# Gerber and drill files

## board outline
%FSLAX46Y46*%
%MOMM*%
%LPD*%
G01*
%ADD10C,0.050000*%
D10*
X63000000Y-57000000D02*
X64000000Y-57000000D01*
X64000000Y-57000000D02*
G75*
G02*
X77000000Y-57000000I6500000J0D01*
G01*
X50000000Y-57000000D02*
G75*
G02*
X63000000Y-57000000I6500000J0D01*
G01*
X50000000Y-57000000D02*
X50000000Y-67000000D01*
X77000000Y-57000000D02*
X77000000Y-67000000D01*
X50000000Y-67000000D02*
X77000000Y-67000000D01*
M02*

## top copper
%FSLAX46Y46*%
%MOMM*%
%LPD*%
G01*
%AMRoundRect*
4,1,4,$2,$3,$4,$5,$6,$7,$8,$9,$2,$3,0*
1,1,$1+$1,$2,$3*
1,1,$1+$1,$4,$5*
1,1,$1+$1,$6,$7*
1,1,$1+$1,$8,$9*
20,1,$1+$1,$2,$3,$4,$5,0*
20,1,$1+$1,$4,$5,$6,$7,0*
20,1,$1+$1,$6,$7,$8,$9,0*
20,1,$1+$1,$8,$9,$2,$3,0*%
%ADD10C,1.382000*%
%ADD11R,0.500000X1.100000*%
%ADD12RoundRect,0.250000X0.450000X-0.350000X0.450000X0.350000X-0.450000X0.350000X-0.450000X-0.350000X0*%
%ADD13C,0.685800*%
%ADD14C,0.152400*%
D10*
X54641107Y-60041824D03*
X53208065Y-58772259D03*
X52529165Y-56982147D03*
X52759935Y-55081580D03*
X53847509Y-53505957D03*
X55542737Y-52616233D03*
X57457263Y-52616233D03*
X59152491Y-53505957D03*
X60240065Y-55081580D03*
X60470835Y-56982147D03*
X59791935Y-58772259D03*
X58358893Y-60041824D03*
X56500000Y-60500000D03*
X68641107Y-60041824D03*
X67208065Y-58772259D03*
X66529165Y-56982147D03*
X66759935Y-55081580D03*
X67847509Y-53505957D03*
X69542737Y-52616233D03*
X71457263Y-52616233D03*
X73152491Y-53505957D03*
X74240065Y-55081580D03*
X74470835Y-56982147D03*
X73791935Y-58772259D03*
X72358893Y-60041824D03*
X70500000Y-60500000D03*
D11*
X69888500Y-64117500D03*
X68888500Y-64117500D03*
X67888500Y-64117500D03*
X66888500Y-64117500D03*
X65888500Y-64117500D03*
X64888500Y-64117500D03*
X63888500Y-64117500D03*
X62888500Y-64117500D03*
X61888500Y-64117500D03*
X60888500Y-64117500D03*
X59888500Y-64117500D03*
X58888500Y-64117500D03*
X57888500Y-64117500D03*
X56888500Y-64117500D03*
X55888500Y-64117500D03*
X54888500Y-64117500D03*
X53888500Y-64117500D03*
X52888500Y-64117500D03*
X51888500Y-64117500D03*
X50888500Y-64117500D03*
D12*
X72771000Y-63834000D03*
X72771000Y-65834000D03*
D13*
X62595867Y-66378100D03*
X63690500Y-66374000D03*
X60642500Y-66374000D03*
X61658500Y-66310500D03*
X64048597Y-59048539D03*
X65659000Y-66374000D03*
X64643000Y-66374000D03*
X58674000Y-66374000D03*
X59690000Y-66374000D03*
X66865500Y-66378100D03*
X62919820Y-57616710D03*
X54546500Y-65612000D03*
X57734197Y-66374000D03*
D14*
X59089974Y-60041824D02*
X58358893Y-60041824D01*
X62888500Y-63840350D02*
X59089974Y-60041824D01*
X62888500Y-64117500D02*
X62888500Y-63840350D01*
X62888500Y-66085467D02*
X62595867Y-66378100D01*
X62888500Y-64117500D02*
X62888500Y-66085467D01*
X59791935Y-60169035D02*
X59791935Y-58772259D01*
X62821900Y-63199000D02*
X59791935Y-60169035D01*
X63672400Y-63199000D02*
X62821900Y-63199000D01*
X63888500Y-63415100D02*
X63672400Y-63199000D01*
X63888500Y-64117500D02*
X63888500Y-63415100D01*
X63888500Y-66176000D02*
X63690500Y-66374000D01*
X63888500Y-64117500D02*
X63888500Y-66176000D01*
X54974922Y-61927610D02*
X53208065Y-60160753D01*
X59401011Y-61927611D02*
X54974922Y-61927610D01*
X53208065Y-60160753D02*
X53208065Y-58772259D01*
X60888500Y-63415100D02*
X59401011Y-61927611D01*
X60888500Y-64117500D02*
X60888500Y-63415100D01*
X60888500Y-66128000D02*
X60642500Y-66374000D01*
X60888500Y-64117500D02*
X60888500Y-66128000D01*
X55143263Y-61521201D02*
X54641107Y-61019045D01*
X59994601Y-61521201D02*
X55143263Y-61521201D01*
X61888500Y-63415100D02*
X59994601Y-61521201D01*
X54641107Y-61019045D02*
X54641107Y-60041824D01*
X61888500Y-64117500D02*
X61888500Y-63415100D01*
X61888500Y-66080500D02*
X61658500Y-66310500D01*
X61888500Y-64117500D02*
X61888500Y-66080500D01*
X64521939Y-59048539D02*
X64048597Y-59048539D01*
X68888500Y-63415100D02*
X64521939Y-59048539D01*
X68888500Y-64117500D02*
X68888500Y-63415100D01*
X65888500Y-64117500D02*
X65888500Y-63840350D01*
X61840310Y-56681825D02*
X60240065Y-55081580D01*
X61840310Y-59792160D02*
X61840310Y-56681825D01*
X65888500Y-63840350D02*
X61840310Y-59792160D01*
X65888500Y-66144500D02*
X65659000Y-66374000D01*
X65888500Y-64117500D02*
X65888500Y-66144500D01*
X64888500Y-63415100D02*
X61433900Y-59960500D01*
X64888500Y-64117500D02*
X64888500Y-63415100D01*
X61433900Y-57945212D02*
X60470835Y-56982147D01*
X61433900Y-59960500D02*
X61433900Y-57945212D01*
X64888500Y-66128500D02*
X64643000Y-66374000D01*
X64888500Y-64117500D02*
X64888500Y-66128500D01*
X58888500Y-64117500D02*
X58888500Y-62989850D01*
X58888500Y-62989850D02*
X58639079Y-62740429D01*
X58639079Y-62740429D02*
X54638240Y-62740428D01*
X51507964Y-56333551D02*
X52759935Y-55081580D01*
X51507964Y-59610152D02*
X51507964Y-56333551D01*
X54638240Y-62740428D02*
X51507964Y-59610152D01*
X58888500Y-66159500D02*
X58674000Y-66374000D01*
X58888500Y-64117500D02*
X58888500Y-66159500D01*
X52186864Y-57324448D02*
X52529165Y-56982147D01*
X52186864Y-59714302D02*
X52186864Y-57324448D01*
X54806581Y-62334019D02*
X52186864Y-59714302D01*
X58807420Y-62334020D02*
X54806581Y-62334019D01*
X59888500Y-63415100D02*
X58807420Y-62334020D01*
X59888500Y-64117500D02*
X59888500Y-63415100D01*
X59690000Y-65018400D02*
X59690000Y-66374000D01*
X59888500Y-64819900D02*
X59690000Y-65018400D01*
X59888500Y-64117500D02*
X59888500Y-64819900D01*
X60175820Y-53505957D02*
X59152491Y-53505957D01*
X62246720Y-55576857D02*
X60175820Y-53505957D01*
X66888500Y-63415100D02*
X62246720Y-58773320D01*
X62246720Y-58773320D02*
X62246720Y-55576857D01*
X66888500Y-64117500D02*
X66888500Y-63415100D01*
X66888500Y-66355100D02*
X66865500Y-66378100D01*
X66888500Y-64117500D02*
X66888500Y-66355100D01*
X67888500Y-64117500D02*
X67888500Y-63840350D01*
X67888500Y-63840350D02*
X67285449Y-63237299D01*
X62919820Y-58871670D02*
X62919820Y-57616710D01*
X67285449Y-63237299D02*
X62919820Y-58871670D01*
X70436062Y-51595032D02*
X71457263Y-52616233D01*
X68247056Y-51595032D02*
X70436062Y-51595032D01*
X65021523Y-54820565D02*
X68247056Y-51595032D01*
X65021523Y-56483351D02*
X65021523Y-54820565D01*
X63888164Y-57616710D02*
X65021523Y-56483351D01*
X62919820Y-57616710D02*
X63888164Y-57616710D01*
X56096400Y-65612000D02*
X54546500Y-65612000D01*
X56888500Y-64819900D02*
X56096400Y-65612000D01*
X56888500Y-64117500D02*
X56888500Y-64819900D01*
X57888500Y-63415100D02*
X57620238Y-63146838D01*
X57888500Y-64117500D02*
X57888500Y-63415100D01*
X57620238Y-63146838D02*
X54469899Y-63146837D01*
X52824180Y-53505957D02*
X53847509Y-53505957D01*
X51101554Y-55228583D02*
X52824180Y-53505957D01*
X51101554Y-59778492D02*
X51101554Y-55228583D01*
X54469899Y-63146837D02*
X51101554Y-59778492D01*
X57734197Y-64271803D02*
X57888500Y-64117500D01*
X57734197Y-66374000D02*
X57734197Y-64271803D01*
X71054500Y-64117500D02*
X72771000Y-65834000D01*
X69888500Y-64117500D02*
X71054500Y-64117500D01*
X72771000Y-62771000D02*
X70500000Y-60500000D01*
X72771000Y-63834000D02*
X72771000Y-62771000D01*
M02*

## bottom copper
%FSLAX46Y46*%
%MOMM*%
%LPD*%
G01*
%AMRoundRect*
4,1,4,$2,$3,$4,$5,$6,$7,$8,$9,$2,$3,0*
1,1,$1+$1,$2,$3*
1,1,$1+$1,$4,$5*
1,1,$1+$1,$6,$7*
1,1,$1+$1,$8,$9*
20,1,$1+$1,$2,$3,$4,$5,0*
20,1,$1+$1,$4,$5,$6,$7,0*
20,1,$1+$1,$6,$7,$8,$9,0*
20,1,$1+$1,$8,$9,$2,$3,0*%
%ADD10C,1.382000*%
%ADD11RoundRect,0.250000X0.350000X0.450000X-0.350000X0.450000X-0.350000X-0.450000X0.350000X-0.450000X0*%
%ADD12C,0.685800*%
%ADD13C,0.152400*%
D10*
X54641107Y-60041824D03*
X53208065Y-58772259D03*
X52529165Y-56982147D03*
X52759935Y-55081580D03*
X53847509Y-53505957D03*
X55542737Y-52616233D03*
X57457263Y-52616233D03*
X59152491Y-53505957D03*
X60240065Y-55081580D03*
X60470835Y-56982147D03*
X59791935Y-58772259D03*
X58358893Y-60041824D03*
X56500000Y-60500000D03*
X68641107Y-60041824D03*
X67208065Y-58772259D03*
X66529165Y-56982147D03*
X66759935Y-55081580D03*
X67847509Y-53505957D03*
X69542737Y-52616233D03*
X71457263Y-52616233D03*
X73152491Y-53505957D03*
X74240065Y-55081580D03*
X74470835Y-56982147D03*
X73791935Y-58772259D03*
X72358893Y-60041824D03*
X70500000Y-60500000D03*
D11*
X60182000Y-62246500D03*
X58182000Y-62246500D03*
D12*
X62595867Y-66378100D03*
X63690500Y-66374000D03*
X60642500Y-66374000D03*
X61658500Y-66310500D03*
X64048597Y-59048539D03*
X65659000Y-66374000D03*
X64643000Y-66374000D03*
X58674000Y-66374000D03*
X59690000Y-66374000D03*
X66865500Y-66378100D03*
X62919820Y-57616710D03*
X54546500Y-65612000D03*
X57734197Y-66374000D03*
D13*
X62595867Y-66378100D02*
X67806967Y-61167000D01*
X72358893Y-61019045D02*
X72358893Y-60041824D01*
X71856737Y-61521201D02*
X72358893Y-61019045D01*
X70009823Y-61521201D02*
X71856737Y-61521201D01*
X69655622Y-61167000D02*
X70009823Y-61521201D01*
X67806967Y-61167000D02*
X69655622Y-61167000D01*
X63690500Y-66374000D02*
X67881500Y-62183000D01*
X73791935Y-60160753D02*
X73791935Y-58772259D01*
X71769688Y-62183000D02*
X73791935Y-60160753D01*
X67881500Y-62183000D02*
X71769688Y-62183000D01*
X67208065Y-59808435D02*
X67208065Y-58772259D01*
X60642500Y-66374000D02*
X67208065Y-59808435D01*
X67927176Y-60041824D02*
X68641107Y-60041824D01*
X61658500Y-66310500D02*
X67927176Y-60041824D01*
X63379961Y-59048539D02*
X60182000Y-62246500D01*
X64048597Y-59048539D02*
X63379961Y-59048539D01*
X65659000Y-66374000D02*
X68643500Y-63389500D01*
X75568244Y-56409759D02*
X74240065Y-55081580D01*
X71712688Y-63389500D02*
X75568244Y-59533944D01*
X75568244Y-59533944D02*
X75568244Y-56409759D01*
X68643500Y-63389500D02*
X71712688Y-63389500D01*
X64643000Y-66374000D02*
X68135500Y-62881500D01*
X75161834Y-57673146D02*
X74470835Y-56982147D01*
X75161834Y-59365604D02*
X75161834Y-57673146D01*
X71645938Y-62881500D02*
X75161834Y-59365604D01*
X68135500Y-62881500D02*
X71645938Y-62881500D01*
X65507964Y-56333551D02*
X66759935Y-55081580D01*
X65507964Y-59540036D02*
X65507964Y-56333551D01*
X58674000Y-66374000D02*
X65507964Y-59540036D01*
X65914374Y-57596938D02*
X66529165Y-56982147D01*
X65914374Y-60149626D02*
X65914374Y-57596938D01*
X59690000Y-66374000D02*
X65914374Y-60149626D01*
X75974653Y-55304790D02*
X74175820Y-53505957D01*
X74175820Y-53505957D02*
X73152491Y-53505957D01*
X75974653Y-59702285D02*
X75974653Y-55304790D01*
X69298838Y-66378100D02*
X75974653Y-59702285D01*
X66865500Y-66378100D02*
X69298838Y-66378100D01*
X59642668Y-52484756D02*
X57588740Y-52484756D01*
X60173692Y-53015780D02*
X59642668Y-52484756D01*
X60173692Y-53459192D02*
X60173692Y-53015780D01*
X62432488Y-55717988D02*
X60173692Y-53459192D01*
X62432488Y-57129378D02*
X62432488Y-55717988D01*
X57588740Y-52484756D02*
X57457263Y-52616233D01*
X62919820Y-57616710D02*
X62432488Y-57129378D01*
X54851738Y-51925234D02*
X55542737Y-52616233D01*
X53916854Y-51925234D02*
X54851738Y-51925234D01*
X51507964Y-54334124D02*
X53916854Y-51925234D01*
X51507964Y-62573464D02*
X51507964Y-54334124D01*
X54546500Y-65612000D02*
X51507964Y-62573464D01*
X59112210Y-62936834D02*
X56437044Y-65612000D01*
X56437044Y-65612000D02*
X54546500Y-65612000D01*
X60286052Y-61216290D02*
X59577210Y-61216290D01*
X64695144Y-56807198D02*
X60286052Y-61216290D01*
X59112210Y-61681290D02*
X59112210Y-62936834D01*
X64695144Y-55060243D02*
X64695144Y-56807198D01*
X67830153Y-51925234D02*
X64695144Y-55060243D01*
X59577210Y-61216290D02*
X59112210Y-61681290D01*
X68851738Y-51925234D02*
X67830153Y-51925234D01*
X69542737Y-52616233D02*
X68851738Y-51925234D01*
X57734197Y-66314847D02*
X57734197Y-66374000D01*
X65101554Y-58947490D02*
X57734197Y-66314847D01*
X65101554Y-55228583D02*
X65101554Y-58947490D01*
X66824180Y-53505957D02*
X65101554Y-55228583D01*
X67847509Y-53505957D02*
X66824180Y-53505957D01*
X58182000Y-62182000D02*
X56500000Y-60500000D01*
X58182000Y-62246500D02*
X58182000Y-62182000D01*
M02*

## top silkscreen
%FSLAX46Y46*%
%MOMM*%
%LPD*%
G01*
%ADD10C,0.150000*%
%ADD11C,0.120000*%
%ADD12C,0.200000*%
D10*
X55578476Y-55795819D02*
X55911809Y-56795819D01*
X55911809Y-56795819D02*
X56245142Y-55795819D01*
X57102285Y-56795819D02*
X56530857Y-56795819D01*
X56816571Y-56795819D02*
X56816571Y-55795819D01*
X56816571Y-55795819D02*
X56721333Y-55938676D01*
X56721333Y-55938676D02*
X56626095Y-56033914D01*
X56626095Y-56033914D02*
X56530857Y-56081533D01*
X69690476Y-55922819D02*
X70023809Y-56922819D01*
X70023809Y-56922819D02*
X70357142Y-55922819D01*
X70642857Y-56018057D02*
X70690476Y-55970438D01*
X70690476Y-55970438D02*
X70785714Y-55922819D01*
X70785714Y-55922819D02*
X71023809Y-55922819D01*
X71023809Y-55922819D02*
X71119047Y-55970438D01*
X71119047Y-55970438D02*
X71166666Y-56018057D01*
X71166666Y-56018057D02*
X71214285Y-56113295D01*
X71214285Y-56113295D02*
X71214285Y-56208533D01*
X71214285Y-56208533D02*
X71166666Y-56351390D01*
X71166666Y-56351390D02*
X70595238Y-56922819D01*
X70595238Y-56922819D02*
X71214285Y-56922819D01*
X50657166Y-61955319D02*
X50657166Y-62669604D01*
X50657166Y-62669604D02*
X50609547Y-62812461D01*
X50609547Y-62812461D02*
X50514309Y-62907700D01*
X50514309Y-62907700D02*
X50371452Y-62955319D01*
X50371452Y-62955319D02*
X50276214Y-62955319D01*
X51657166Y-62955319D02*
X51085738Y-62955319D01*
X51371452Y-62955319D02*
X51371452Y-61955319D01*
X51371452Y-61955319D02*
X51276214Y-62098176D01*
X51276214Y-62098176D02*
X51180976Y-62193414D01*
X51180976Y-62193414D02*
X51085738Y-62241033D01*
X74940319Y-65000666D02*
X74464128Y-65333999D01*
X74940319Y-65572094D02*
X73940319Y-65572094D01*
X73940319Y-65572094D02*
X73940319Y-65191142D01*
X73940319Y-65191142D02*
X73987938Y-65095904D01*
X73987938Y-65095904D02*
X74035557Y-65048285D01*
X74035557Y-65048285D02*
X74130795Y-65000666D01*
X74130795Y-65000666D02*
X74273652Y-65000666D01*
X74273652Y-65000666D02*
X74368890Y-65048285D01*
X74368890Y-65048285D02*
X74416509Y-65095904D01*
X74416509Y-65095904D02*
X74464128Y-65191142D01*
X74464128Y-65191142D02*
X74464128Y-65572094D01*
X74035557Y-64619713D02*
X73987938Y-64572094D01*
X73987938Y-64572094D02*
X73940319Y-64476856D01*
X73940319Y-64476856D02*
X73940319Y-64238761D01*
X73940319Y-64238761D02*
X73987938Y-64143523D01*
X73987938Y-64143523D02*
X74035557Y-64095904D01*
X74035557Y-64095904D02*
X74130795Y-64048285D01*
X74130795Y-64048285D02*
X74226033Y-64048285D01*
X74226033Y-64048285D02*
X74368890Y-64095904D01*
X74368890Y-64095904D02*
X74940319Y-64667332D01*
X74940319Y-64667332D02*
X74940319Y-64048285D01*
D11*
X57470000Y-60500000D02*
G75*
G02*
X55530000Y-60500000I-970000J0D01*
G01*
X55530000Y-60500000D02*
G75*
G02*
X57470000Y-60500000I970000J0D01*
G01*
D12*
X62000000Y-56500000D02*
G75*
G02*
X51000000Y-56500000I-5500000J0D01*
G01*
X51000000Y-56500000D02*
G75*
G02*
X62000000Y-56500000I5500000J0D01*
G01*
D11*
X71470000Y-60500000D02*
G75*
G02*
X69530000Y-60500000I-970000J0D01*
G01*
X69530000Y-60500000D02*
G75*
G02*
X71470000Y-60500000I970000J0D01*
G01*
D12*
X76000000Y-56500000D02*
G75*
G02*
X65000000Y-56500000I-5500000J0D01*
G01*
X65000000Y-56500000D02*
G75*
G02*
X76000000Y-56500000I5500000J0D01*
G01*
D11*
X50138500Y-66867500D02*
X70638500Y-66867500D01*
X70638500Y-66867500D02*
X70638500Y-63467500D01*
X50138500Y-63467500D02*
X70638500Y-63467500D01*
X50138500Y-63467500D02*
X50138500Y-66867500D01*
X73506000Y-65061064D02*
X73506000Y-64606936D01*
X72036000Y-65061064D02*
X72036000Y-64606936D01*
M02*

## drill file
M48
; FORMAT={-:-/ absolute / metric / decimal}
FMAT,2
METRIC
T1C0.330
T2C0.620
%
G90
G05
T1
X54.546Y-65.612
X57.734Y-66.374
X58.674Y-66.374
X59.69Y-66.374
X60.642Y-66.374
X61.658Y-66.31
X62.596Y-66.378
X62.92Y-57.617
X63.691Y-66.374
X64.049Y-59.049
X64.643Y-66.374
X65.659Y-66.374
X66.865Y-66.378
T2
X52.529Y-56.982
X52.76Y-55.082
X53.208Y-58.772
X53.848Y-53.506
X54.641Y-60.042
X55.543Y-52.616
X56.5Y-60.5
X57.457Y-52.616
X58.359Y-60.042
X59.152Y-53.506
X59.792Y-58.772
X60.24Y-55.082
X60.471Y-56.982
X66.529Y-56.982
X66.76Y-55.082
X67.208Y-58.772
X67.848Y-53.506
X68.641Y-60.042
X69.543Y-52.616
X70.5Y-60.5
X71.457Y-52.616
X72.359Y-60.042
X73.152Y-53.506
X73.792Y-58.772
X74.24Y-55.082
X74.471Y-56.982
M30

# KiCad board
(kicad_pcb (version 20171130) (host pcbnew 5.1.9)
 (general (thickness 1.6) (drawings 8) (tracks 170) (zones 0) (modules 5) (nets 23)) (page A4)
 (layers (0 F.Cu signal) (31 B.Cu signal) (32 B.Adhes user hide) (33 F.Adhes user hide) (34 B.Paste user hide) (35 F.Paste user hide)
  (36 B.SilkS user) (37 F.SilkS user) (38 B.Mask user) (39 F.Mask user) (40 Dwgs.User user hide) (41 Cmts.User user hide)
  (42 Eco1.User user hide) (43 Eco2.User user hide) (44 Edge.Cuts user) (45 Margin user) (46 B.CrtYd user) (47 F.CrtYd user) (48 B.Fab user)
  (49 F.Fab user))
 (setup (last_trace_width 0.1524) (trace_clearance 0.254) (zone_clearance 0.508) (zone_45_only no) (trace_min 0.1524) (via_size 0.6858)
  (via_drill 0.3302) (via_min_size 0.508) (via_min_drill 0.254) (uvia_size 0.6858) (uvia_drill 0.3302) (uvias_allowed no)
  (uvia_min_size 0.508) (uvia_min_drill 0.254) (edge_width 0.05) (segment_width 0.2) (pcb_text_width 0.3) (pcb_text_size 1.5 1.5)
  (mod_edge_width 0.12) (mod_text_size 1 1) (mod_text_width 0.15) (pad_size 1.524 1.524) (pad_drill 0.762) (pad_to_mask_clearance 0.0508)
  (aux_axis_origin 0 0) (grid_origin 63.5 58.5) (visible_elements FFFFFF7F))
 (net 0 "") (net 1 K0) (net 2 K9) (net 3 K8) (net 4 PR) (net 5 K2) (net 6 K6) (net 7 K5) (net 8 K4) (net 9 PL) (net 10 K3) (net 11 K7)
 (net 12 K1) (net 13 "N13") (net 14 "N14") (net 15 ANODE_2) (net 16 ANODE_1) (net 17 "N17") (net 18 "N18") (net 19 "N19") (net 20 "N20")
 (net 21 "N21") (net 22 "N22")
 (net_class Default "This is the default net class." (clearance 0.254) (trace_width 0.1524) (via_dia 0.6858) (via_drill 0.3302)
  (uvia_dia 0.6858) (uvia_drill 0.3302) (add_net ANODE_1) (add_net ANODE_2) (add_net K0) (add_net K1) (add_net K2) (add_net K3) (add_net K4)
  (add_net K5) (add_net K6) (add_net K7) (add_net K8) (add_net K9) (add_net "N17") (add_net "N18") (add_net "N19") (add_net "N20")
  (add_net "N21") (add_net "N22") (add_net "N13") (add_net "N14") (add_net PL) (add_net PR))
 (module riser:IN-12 (layer F.Cu) (at 56.5 56.5)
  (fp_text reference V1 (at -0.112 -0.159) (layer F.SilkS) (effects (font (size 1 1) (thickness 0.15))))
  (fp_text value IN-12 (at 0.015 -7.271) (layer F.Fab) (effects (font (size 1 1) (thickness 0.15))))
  (fp_circle (center 0 4) (end 0.97 4) (layer F.SilkS) (width 0.12))
  (fp_circle (center 0 0) (end 5.5 0) (layer F.SilkS) (width 0.2))
  (pad 13 thru_hole circle (at -1.858893 3.541824) (size 1.382 1.382) (drill 0.62) (layers *.Cu *.Mask) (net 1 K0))
  (pad 12 thru_hole circle (at -3.291935 2.272259) (size 1.382 1.382) (drill 0.62) (layers *.Cu *.Mask) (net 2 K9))
  (pad 11 thru_hole circle (at -3.970835 0.482147) (size 1.382 1.382) (drill 0.62) (layers *.Cu *.Mask) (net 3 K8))
  (pad 10 thru_hole circle (at -3.740065 -1.41842) (size 1.382 1.382) (drill 0.62) (layers *.Cu *.Mask) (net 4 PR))
  (pad 9 thru_hole circle (at -2.652491 -2.994043) (size 1.382 1.382) (drill 0.62) (layers *.Cu *.Mask) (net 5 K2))
  (pad 8 thru_hole circle (at -0.957263 -3.883767) (size 1.382 1.382) (drill 0.62) (layers *.Cu *.Mask) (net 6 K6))
  (pad 7 thru_hole circle (at 0.957263 -3.883767) (size 1.382 1.382) (drill 0.62) (layers *.Cu *.Mask) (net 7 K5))
  (pad 6 thru_hole circle (at 2.652491 -2.994043) (size 1.382 1.382) (drill 0.62) (layers *.Cu *.Mask) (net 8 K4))
  (pad 5 thru_hole circle (at 3.740065 -1.41842) (size 1.382 1.382) (drill 0.62) (layers *.Cu *.Mask) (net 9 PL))
  (pad 4 thru_hole circle (at 3.970835 0.482147) (size 1.382 1.382) (drill 0.62) (layers *.Cu *.Mask) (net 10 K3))
  (pad 3 thru_hole circle (at 3.291935 2.272259) (size 1.382 1.382) (drill 0.62) (layers *.Cu *.Mask) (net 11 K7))
  (pad 2 thru_hole circle (at 1.858893 3.541824) (size 1.382 1.382) (drill 0.62) (layers *.Cu *.Mask) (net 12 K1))
  (pad 1 thru_hole circle (at 0 4) (size 1.382 1.382) (drill 0.62) (layers *.Cu *.Mask) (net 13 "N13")))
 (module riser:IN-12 (layer F.Cu) (at 70.5 56.5)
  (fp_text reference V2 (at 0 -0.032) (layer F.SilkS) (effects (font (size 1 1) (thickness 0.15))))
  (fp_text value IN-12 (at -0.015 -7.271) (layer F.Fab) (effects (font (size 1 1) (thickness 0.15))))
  (fp_circle (center 0 4) (end 0.97 4) (layer F.SilkS) (width 0.12))
  (fp_circle (center 0 0) (end 5.5 0) (layer F.SilkS) (width 0.2))
  (pad 13 thru_hole circle (at -1.858893 3.541824) (size 1.382 1.382) (drill 0.62) (layers *.Cu *.Mask) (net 1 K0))
  (pad 12 thru_hole circle (at -3.291935 2.272259) (size 1.382 1.382) (drill 0.62) (layers *.Cu *.Mask) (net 2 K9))
  (pad 11 thru_hole circle (at -3.970835 0.482147) (size 1.382 1.382) (drill 0.62) (layers *.Cu *.Mask) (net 3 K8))
  (pad 10 thru_hole circle (at -3.740065 -1.41842) (size 1.382 1.382) (drill 0.62) (layers *.Cu *.Mask) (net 4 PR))
  (pad 9 thru_hole circle (at -2.652491 -2.994043) (size 1.382 1.382) (drill 0.62) (layers *.Cu *.Mask) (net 5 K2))
  (pad 8 thru_hole circle (at -0.957263 -3.883767) (size 1.382 1.382) (drill 0.62) (layers *.Cu *.Mask) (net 6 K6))
  (pad 7 thru_hole circle (at 0.957263 -3.883767) (size 1.382 1.382) (drill 0.62) (layers *.Cu *.Mask) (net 7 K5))
  (pad 6 thru_hole circle (at 2.652491 -2.994043) (size 1.382 1.382) (drill 0.62) (layers *.Cu *.Mask) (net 8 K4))
  (pad 5 thru_hole circle (at 3.740065 -1.41842) (size 1.382 1.382) (drill 0.62) (layers *.Cu *.Mask) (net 9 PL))
  (pad 4 thru_hole circle (at 3.970835 0.482147) (size 1.382 1.382) (drill 0.62) (layers *.Cu *.Mask) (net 10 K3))
  (pad 3 thru_hole circle (at 3.291935 2.272259) (size 1.382 1.382) (drill 0.62) (layers *.Cu *.Mask) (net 11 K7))
  (pad 2 thru_hole circle (at 1.858893 3.541824) (size 1.382 1.382) (drill 0.62) (layers *.Cu *.Mask) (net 12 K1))
  (pad 1 thru_hole circle (at 0 4) (size 1.382 1.382) (drill 0.62) (layers *.Cu *.Mask) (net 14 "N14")))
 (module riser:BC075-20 (layer F.Cu) (at 60.3885 65.1675)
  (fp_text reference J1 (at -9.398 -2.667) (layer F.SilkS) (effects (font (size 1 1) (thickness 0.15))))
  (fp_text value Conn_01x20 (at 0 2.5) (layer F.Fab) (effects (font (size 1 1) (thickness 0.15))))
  (fp_line (start -10.25 1.7) (end 10.25 1.7) (layer F.SilkS) (width 0.12))
  (fp_line (start 10.25 1.7) (end 10.25 -1.7) (layer F.SilkS) (width 0.12))
  (fp_line (start -10.25 -1.7) (end 10.25 -1.7) (layer F.SilkS) (width 0.12))
  (fp_line (start -10.25 -1.7) (end -10.25 1.7) (layer F.SilkS) (width 0.12))
  (pad 1 smd rect (at 9.5 -1.05) (size 0.5 1.1) (layers F.Cu F.Paste F.Mask) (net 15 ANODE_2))
  (pad 2 smd rect (at 8.5 -1.05) (size 0.5 1.1) (layers F.Cu F.Paste F.Mask) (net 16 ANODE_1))
  (pad 3 smd rect (at 7.5 -1.05) (size 0.5 1.1) (layers F.Cu F.Paste F.Mask) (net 7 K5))
  (pad 4 smd rect (at 6.5 -1.05) (size 0.5 1.1) (layers F.Cu F.Paste F.Mask) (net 8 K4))
  (pad 5 smd rect (at 5.5 -1.05) (size 0.5 1.1) (layers F.Cu F.Paste F.Mask) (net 9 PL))
  (pad 6 smd rect (at 4.5 -1.05) (size 0.5 1.1) (layers F.Cu F.Paste F.Mask) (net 10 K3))
  (pad 7 smd rect (at 3.5 -1.05) (size 0.5 1.1) (layers F.Cu F.Paste F.Mask) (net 11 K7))
  (pad 8 smd rect (at 2.5 -1.05) (size 0.5 1.1) (layers F.Cu F.Paste F.Mask) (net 12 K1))
  (pad 9 smd rect (at 1.5 -1.05) (size 0.5 1.1) (layers F.Cu F.Paste F.Mask) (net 1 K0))
  (pad 10 smd rect (at 0.5 -1.05) (size 0.5 1.1) (layers F.Cu F.Paste F.Mask) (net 2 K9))
  (pad 11 smd rect (at -0.5 -1.05) (size 0.5 1.1) (layers F.Cu F.Paste F.Mask) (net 3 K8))
  (pad 12 smd rect (at -1.5 -1.05) (size 0.5 1.1) (layers F.Cu F.Paste F.Mask) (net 4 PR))
  (pad 13 smd rect (at -2.5 -1.05) (size 0.5 1.1) (layers F.Cu F.Paste F.Mask) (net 5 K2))
  (pad 14 smd rect (at -3.5 -1.05) (size 0.5 1.1) (layers F.Cu F.Paste F.Mask) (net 6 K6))
  (pad 15 smd rect (at -4.5 -1.05) (size 0.5 1.1) (layers F.Cu F.Paste F.Mask) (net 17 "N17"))
  (pad 16 smd rect (at -5.5 -1.05) (size 0.5 1.1) (layers F.Cu F.Paste F.Mask) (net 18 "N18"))
  (pad 17 smd rect (at -6.5 -1.05) (size 0.5 1.1) (layers F.Cu F.Paste F.Mask) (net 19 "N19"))
  (pad 18 smd rect (at -7.5 -1.05) (size 0.5 1.1) (layers F.Cu F.Paste F.Mask) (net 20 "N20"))
  (pad 19 smd rect (at -8.5 -1.05) (size 0.5 1.1) (layers F.Cu F.Paste F.Mask) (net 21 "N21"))
  (pad 20 smd rect (at -9.5 -1.05) (size 0.5 1.1) (layers F.Cu F.Paste F.Mask) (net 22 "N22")))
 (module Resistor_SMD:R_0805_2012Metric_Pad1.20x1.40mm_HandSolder (layer B.Cu) (at 59.182 62.2465 180)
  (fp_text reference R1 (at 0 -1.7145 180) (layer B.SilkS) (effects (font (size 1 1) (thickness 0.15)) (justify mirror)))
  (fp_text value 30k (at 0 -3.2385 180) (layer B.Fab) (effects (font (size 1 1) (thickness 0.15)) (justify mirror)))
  (pad 1 smd roundrect (at -1 0 180) (size 1.2 1.4) (layers B.Cu B.Paste B.Mask) (roundrect_rratio 0.208333) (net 16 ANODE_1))
  (pad 2 smd roundrect (at 1 0 180) (size 1.2 1.4) (layers B.Cu B.Paste B.Mask) (roundrect_rratio 0.208333) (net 13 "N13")))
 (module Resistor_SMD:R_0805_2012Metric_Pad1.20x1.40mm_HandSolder (layer F.Cu) (at 72.771 64.834 90)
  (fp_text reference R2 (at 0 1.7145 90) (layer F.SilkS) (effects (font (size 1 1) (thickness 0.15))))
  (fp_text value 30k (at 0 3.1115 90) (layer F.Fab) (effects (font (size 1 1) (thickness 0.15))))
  (fp_line (start -0.227064 0.735) (end 0.227064 0.735) (layer F.SilkS) (width 0.12))
  (fp_line (start -0.227064 -0.735) (end 0.227064 -0.735) (layer F.SilkS) (width 0.12))
  (pad 2 smd roundrect (at 1 0 90) (size 1.2 1.4) (layers F.Cu F.Paste F.Mask) (roundrect_rratio 0.208333) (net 14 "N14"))
  (pad 1 smd roundrect (at -1 0 90) (size 1.2 1.4) (layers F.Cu F.Paste F.Mask) (roundrect_rratio 0.208333) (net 15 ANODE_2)))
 (gr_line (start 63 57) (end 64 57) (layer Edge.Cuts) (width 0.05))
 (gr_arc (start 70.5 57) (end 77 57) (angle -180) (layer Edge.Cuts) (width 0.05))
 (gr_arc (start 56.5 57) (end 50 57) (angle 180) (layer Edge.Cuts) (width 0.05))
 (gr_line (start 50 57) (end 50 67) (layer Edge.Cuts) (width 0.05))
 (gr_line (start 77 57) (end 77 67) (layer Edge.Cuts) (width 0.05))
 (gr_line (start 50 67) (end 77 67) (layer Edge.Cuts) (width 0.05))
 (segment (start 59.089974 60.041824) (end 58.358893 60.041824) (width 0.1524) (layer F.Cu) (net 12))
 (segment (start 62.8885 63.84035) (end 59.089974 60.041824) (width 0.1524) (layer F.Cu) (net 12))
 (segment (start 62.8885 64.1175) (end 62.8885 63.84035) (width 0.1524) (layer F.Cu) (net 12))
 (via (at 62.595867 66.3781) (size 0.6858) (drill 0.3302) (layers F.Cu B.Cu) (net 12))
 (segment (start 62.8885 66.085467) (end 62.595867 66.3781) (width 0.1524) (layer F.Cu) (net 12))
 (segment (start 62.8885 64.1175) (end 62.8885 66.085467) (width 0.1524) (layer F.Cu) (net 12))
 (segment (start 62.595867 66.3781) (end 67.806967 61.167) (width 0.1524) (layer B.Cu) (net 12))
 (segment (start 72.358893 61.019045) (end 72.358893 60.041824) (width 0.1524) (layer B.Cu) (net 12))
 (segment (start 71.856737 61.521201) (end 72.358893 61.019045) (width 0.1524) (layer B.Cu) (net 12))
 (segment (start 70.009823 61.521201) (end 71.856737 61.521201) (width 0.1524) (layer B.Cu) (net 12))
 (segment (start 69.655622 61.167) (end 70.009823 61.521201) (width 0.1524) (layer B.Cu) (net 12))
 (segment (start 67.806967 61.167) (end 69.655622 61.167) (width 0.1524) (layer B.Cu) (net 12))
 (segment (start 59.791935 60.169035) (end 59.791935 58.772259) (width 0.1524) (layer F.Cu) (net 11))
 (segment (start 62.8219 63.199) (end 59.791935 60.169035) (width 0.1524) (layer F.Cu) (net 11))
 (segment (start 63.6724 63.199) (end 62.8219 63.199) (width 0.1524) (layer F.Cu) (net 11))
 (segment (start 63.8885 63.4151) (end 63.6724 63.199) (width 0.1524) (layer F.Cu) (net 11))
 (segment (start 63.8885 64.1175) (end 63.8885 63.4151) (width 0.1524) (layer F.Cu) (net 11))
 (via (at 63.6905 66.374) (size 0.6858) (drill 0.3302) (layers F.Cu B.Cu) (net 11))
 (segment (start 63.8885 66.176) (end 63.6905 66.374) (width 0.1524) (layer F.Cu) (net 11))
 (segment (start 63.8885 64.1175) (end 63.8885 66.176) (width 0.1524) (layer F.Cu) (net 11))
 (segment (start 63.6905 66.374) (end 67.8815 62.183) (width 0.1524) (layer B.Cu) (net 11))
 (segment (start 73.791935 60.160753) (end 73.791935 58.772259) (width 0.1524) (layer B.Cu) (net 11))
 (segment (start 71.769688 62.183) (end 73.791935 60.160753) (width 0.1524) (layer B.Cu) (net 11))
 (segment (start 67.8815 62.183) (end 71.769688 62.183) (width 0.1524) (layer B.Cu) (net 11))
 (segment (start 54.974922 61.92761) (end 53.208065 60.160753) (width 0.1524) (layer F.Cu) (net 2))
 (segment (start 59.401011 61.927611) (end 54.974922 61.92761) (width 0.1524) (layer F.Cu) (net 2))
 (segment (start 53.208065 60.160753) (end 53.208065 58.772259) (width 0.1524) (layer F.Cu) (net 2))
 (segment (start 60.8885 63.4151) (end 59.401011 61.927611) (width 0.1524) (layer F.Cu) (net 2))
 (segment (start 60.8885 64.1175) (end 60.8885 63.4151) (width 0.1524) (layer F.Cu) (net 2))
 (via (at 60.6425 66.374) (size 0.6858) (drill 0.3302) (layers F.Cu B.Cu) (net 2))
 (segment (start 60.8885 66.128) (end 60.6425 66.374) (width 0.1524) (layer F.Cu) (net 2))
 (segment (start 60.8885 64.1175) (end 60.8885 66.128) (width 0.1524) (layer F.Cu) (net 2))
 (segment (start 67.208065 59.808435) (end 67.208065 58.772259) (width 0.1524) (layer B.Cu) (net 2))
 (segment (start 60.6425 66.374) (end 67.208065 59.808435) (width 0.1524) (layer B.Cu) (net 2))
 (segment (start 55.143263 61.521201) (end 54.641107 61.019045) (width 0.1524) (layer F.Cu) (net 1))
 (segment (start 59.994601 61.521201) (end 55.143263 61.521201) (width 0.1524) (layer F.Cu) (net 1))
 (segment (start 61.8885 63.4151) (end 59.994601 61.521201) (width 0.1524) (layer F.Cu) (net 1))
 (segment (start 54.641107 61.019045) (end 54.641107 60.041824) (width 0.1524) (layer F.Cu) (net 1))
 (segment (start 61.8885 64.1175) (end 61.8885 63.4151) (width 0.1524) (layer F.Cu) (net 1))
 (via (at 61.6585 66.3105) (size 0.6858) (drill 0.3302) (layers F.Cu B.Cu) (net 1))
 (segment (start 61.8885 66.0805) (end 61.6585 66.3105) (width 0.1524) (layer F.Cu) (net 1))
 (segment (start 61.8885 64.1175) (end 61.8885 66.0805) (width 0.1524) (layer F.Cu) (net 1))
 (segment (start 67.927176 60.041824) (end 68.641107 60.041824) (width 0.1524) (layer B.Cu) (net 1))
 (segment (start 61.6585 66.3105) (end 67.927176 60.041824) (width 0.1524) (layer B.Cu) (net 1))
 (via (at 64.048597 59.048539) (size 0.6858) (drill 0.3302) (layers F.Cu B.Cu) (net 16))
 (segment (start 64.521939 59.048539) (end 64.048597 59.048539) (width 0.1524) (layer F.Cu) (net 16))
 (segment (start 68.8885 63.4151) (end 64.521939 59.048539) (width 0.1524) (layer F.Cu) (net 16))
 (segment (start 68.8885 64.1175) (end 68.8885 63.4151) (width 0.1524) (layer F.Cu) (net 16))
 (segment (start 63.379961 59.048539) (end 60.182 62.2465) (width 0.1524) (layer B.Cu) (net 16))
 (segment (start 64.048597 59.048539) (end 63.379961 59.048539) (width 0.1524) (layer B.Cu) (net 16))
 (segment (start 65.8885 64.1175) (end 65.8885 63.84035) (width 0.1524) (layer F.Cu) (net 9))
 (segment (start 61.84031 56.681825) (end 60.240065 55.08158) (width 0.1524) (layer F.Cu) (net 9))
 (segment (start 61.84031 59.79216) (end 61.84031 56.681825) (width 0.1524) (layer F.Cu) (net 9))
 (segment (start 65.8885 63.84035) (end 61.84031 59.79216) (width 0.1524) (layer F.Cu) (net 9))
 (via (at 65.659 66.374) (size 0.6858) (drill 0.3302) (layers F.Cu B.Cu) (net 9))
 (segment (start 65.8885 66.1445) (end 65.659 66.374) (width 0.1524) (layer F.Cu) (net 9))
 (segment (start 65.8885 64.1175) (end 65.8885 66.1445) (width 0.1524) (layer F.Cu) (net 9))
 (segment (start 65.659 66.374) (end 68.6435 63.3895) (width 0.1524) (layer B.Cu) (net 9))
 (segment (start 75.568244 56.409759) (end 74.240065 55.08158) (width 0.1524) (layer B.Cu) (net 9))
 (segment (start 71.712688 63.3895) (end 75.568244 59.533944) (width 0.1524) (layer B.Cu) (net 9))
 (segment (start 75.568244 59.533944) (end 75.568244 56.409759) (width 0.1524) (layer B.Cu) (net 9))
 (segment (start 68.6435 63.3895) (end 71.712688 63.3895) (width 0.1524) (layer B.Cu) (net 9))
 (segment (start 64.8885 63.4151) (end 61.4339 59.9605) (width 0.1524) (layer F.Cu) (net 10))
 (segment (start 64.8885 64.1175) (end 64.8885 63.4151) (width 0.1524) (layer F.Cu) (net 10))
 (segment (start 61.4339 57.945212) (end 60.470835 56.982147) (width 0.1524) (layer F.Cu) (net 10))
 (segment (start 61.4339 59.9605) (end 61.4339 57.945212) (width 0.1524) (layer F.Cu) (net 10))
 (via (at 64.643 66.374) (size 0.6858) (drill 0.3302) (layers F.Cu B.Cu) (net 10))
 (segment (start 64.8885 66.1285) (end 64.643 66.374) (width 0.1524) (layer F.Cu) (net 10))
 (segment (start 64.8885 64.1175) (end 64.8885 66.1285) (width 0.1524) (layer F.Cu) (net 10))
 (segment (start 64.643 66.374) (end 68.1355 62.8815) (width 0.1524) (layer B.Cu) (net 10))
 (segment (start 75.161834 57.673146) (end 74.470835 56.982147) (width 0.1524) (layer B.Cu) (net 10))
 (segment (start 75.161834 59.365604) (end 75.161834 57.673146) (width 0.1524) (layer B.Cu) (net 10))
 (segment (start 71.645938 62.8815) (end 75.161834 59.365604) (width 0.1524) (layer B.Cu) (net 10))
 (segment (start 68.1355 62.8815) (end 71.645938 62.8815) (width 0.1524) (layer B.Cu) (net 10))
 (segment (start 58.8885 64.1175) (end 58.8885 62.98985) (width 0.1524) (layer F.Cu) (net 4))
 (segment (start 58.8885 62.98985) (end 58.639079 62.740429) (width 0.1524) (layer F.Cu) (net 4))
 (segment (start 58.639079 62.740429) (end 54.63824 62.740428) (width 0.1524) (layer F.Cu) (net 4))
 (segment (start 51.507964 56.333551) (end 52.759935 55.08158) (width 0.1524) (layer F.Cu) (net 4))
 (segment (start 51.507964 59.610152) (end 51.507964 56.333551) (width 0.1524) (layer F.Cu) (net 4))
 (segment (start 54.63824 62.740428) (end 51.507964 59.610152) (width 0.1524) (layer F.Cu) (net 4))
 (segment (start 58.8885 66.1595) (end 58.674 66.374) (width 0.1524) (layer F.Cu) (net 4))
 (via (at 58.674 66.374) (size 0.6858) (drill 0.3302) (layers F.Cu B.Cu) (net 4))
 (segment (start 58.8885 64.1175) (end 58.8885 66.1595) (width 0.1524) (layer F.Cu) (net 4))
 (segment (start 65.507964 56.333551) (end 66.759935 55.08158) (width 0.1524) (layer B.Cu) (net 4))
 (segment (start 65.507964 59.540036) (end 65.507964 56.333551) (width 0.1524) (layer B.Cu) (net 4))
 (segment (start 58.674 66.374) (end 65.507964 59.540036) (width 0.1524) (layer B.Cu) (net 4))
 (segment (start 52.186864 57.324448) (end 52.529165 56.982147) (width 0.1524) (layer F.Cu) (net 3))
 (segment (start 52.186864 59.714302) (end 52.186864 57.324448) (width 0.1524) (layer F.Cu) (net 3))
 (segment (start 54.806581 62.334019) (end 52.186864 59.714302) (width 0.1524) (layer F.Cu) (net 3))
 (segment (start 58.80742 62.33402) (end 54.806581 62.334019) (width 0.1524) (layer F.Cu) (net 3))
 (segment (start 59.8885 63.4151) (end 58.80742 62.33402) (width 0.1524) (layer F.Cu) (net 3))
 (segment (start 59.8885 64.1175) (end 59.8885 63.4151) (width 0.1524) (layer F.Cu) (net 3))
 (segment (start 59.69 65.0184) (end 59.69 66.374) (width 0.1524) (layer F.Cu) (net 3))
 (segment (start 59.8885 64.8199) (end 59.69 65.0184) (width 0.1524) (layer F.Cu) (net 3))
 (via (at 59.69 66.374) (size 0.6858) (drill 0.3302) (layers F.Cu B.Cu) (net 3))
 (segment (start 59.8885 64.1175) (end 59.8885 64.8199) (width 0.1524) (layer F.Cu) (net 3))
 (segment (start 65.914374 57.596938) (end 66.529165 56.982147) (width 0.1524) (layer B.Cu) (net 3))
 (segment (start 65.914374 60.149626) (end 65.914374 57.596938) (width 0.1524) (layer B.Cu) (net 3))
 (segment (start 59.69 66.374) (end 65.914374 60.149626) (width 0.1524) (layer B.Cu) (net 3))
 (segment (start 60.17582 53.505957) (end 59.152491 53.505957) (width 0.1524) (layer F.Cu) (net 8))
 (segment (start 62.24672 55.576857) (end 60.17582 53.505957) (width 0.1524) (layer F.Cu) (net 8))
 (segment (start 66.8885 63.4151) (end 62.24672 58.77332) (width 0.1524) (layer F.Cu) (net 8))
 (segment (start 62.24672 58.77332) (end 62.24672 55.576857) (width 0.1524) (layer F.Cu) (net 8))
 (segment (start 66.8885 64.1175) (end 66.8885 63.4151) (width 0.1524) (layer F.Cu) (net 8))
 (via (at 66.8655 66.3781) (size 0.6858) (drill 0.3302) (layers F.Cu B.Cu) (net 8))
 (segment (start 66.8885 66.3551) (end 66.8655 66.3781) (width 0.1524) (layer F.Cu) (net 8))
 (segment (start 66.8885 64.1175) (end 66.8885 66.3551) (width 0.1524) (layer F.Cu) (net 8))
 (segment (start 75.974653 55.30479) (end 74.17582 53.505957) (width 0.1524) (layer B.Cu) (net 8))
 (segment (start 74.17582 53.505957) (end 73.152491 53.505957) (width 0.1524) (layer B.Cu) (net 8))
 (segment (start 75.974653 59.702285) (end 75.974653 55.30479) (width 0.1524) (layer B.Cu) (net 8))
 (segment (start 69.298838 66.3781) (end 75.974653 59.702285) (width 0.1524) (layer B.Cu) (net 8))
 (segment (start 66.8655 66.3781) (end 69.298838 66.3781) (width 0.1524) (layer B.Cu) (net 8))
 (segment (start 67.8885 64.1175) (end 67.8885 63.84035) (width 0.1524) (layer F.Cu) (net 7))
 (segment (start 67.8885 63.84035) (end 67.285449 63.237299) (width 0.1524) (layer F.Cu) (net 7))
 (via (at 62.91982 57.61671) (size 0.6858) (drill 0.3302) (layers F.Cu B.Cu) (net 7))
 (segment (start 62.91982 58.87167) (end 62.91982 57.61671) (width 0.1524) (layer F.Cu) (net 7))
 (segment (start 67.285449 63.237299) (end 62.91982 58.87167) (width 0.1524) (layer F.Cu) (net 7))
 (segment (start 59.642668 52.484756) (end 57.58874 52.484756) (width 0.1524) (layer B.Cu) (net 7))
 (segment (start 60.173692 53.01578) (end 59.642668 52.484756) (width 0.1524) (layer B.Cu) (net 7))
 (segment (start 60.173692 53.459192) (end 60.173692 53.01578) (width 0.1524) (layer B.Cu) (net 7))
 (segment (start 62.432488 55.717988) (end 60.173692 53.459192) (width 0.1524) (layer B.Cu) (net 7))
 (segment (start 62.432488 57.129378) (end 62.432488 55.717988) (width 0.1524) (layer B.Cu) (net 7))
 (segment (start 57.58874 52.484756) (end 57.457263 52.616233) (width 0.1524) (layer B.Cu) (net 7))
 (segment (start 62.91982 57.61671) (end 62.432488 57.129378) (width 0.1524) (layer B.Cu) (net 7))
 (segment (start 70.436062 51.595032) (end 71.457263 52.616233) (width 0.1524) (layer F.Cu) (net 7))
 (segment (start 68.247056 51.595032) (end 70.436062 51.595032) (width 0.1524) (layer F.Cu) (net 7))
 (segment (start 65.021523 54.820565) (end 68.247056 51.595032) (width 0.1524) (layer F.Cu) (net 7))
 (segment (start 65.021523 56.483351) (end 65.021523 54.820565) (width 0.1524) (layer F.Cu) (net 7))
 (segment (start 63.888164 57.61671) (end 65.021523 56.483351) (width 0.1524) (layer F.Cu) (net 7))
 (segment (start 62.91982 57.61671) (end 63.888164 57.61671) (width 0.1524) (layer F.Cu) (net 7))
 (via (at 54.5465 65.612) (size 0.6858) (drill 0.3302) (layers F.Cu B.Cu) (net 6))
 (segment (start 56.0964 65.612) (end 54.5465 65.612) (width 0.1524) (layer F.Cu) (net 6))
 (segment (start 56.8885 64.8199) (end 56.0964 65.612) (width 0.1524) (layer F.Cu) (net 6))
 (segment (start 56.8885 64.1175) (end 56.8885 64.8199) (width 0.1524) (layer F.Cu) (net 6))
 (segment (start 54.851738 51.925234) (end 55.542737 52.616233) (width 0.1524) (layer B.Cu) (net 6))
 (segment (start 53.916854 51.925234) (end 54.851738 51.925234) (width 0.1524) (layer B.Cu) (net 6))
 (segment (start 51.507964 54.334124) (end 53.916854 51.925234) (width 0.1524) (layer B.Cu) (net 6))
 (segment (start 51.507964 62.573464) (end 51.507964 54.334124) (width 0.1524) (layer B.Cu) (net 6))
 (segment (start 54.5465 65.612) (end 51.507964 62.573464) (width 0.1524) (layer B.Cu) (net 6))
 (segment (start 59.11221 62.936834) (end 56.437044 65.612) (width 0.1524) (layer B.Cu) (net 6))
 (segment (start 56.437044 65.612) (end 54.5465 65.612) (width 0.1524) (layer B.Cu) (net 6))
 (segment (start 60.286052 61.21629) (end 59.57721 61.21629) (width 0.1524) (layer B.Cu) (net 6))
 (segment (start 64.695144 56.807198) (end 60.286052 61.21629) (width 0.1524) (layer B.Cu) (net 6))
 (segment (start 59.11221 61.68129) (end 59.11221 62.936834) (width 0.1524) (layer B.Cu) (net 6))
 (segment (start 64.695144 55.060243) (end 64.695144 56.807198) (width 0.1524) (layer B.Cu) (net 6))
 (segment (start 67.830153 51.925234) (end 64.695144 55.060243) (width 0.1524) (layer B.Cu) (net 6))
 (segment (start 59.57721 61.21629) (end 59.11221 61.68129) (width 0.1524) (layer B.Cu) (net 6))
 (segment (start 68.851738 51.925234) (end 67.830153 51.925234) (width 0.1524) (layer B.Cu) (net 6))
 (segment (start 69.542737 52.616233) (end 68.851738 51.925234) (width 0.1524) (layer B.Cu) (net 6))
 (segment (start 57.8885 63.4151) (end 57.620238 63.146838) (width 0.1524) (layer F.Cu) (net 5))
 (segment (start 57.8885 64.1175) (end 57.8885 63.4151) (width 0.1524) (layer F.Cu) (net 5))
 (segment (start 57.620238 63.146838) (end 54.469899 63.146837) (width 0.1524) (layer F.Cu) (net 5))
 (segment (start 52.82418 53.505957) (end 53.847509 53.505957) (width 0.1524) (layer F.Cu) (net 5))
 (segment (start 51.101554 55.228583) (end 52.82418 53.505957) (width 0.1524) (layer F.Cu) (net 5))
 (segment (start 51.101554 59.778492) (end 51.101554 55.228583) (width 0.1524) (layer F.Cu) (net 5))
 (segment (start 54.469899 63.146837) (end 51.101554 59.778492) (width 0.1524) (layer F.Cu) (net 5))
 (via (at 57.734197 66.374) (size 0.6858) (drill 0.3302) (layers F.Cu B.Cu) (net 5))
 (segment (start 57.734197 66.314847) (end 57.734197 66.374) (width 0.1524) (layer B.Cu) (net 5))
 (segment (start 65.101554 58.94749) (end 57.734197 66.314847) (width 0.1524) (layer B.Cu) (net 5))
 (segment (start 65.101554 55.228583) (end 65.101554 58.94749) (width 0.1524) (layer B.Cu) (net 5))
 (segment (start 66.82418 53.505957) (end 65.101554 55.228583) (width 0.1524) (layer B.Cu) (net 5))
 (segment (start 67.847509 53.505957) (end 66.82418 53.505957) (width 0.1524) (layer B.Cu) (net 5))
 (segment (start 57.734197 64.271803) (end 57.8885 64.1175) (width 0.1524) (layer F.Cu) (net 5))
 (segment (start 57.734197 66.374) (end 57.734197 64.271803) (width 0.1524) (layer F.Cu) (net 5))
 (segment (start 71.0545 64.1175) (end 72.771 65.834) (width 0.1524) (layer F.Cu) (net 15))
 (segment (start 69.8885 64.1175) (end 71.0545 64.1175) (width 0.1524) (layer F.Cu) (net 15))
 (segment (start 58.182 62.182) (end 56.5 60.5) (width 0.1524) (layer B.Cu) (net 13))
 (segment (start 58.182 62.2465) (end 58.182 62.182) (width 0.1524) (layer B.Cu) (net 13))
 (segment (start 72.771 62.771) (end 70.5 60.5) (width 0.1524) (layer F.Cu) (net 14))
 (segment (start 72.771 63.834) (end 72.771 62.771) (width 0.1524) (layer F.Cu) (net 14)))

